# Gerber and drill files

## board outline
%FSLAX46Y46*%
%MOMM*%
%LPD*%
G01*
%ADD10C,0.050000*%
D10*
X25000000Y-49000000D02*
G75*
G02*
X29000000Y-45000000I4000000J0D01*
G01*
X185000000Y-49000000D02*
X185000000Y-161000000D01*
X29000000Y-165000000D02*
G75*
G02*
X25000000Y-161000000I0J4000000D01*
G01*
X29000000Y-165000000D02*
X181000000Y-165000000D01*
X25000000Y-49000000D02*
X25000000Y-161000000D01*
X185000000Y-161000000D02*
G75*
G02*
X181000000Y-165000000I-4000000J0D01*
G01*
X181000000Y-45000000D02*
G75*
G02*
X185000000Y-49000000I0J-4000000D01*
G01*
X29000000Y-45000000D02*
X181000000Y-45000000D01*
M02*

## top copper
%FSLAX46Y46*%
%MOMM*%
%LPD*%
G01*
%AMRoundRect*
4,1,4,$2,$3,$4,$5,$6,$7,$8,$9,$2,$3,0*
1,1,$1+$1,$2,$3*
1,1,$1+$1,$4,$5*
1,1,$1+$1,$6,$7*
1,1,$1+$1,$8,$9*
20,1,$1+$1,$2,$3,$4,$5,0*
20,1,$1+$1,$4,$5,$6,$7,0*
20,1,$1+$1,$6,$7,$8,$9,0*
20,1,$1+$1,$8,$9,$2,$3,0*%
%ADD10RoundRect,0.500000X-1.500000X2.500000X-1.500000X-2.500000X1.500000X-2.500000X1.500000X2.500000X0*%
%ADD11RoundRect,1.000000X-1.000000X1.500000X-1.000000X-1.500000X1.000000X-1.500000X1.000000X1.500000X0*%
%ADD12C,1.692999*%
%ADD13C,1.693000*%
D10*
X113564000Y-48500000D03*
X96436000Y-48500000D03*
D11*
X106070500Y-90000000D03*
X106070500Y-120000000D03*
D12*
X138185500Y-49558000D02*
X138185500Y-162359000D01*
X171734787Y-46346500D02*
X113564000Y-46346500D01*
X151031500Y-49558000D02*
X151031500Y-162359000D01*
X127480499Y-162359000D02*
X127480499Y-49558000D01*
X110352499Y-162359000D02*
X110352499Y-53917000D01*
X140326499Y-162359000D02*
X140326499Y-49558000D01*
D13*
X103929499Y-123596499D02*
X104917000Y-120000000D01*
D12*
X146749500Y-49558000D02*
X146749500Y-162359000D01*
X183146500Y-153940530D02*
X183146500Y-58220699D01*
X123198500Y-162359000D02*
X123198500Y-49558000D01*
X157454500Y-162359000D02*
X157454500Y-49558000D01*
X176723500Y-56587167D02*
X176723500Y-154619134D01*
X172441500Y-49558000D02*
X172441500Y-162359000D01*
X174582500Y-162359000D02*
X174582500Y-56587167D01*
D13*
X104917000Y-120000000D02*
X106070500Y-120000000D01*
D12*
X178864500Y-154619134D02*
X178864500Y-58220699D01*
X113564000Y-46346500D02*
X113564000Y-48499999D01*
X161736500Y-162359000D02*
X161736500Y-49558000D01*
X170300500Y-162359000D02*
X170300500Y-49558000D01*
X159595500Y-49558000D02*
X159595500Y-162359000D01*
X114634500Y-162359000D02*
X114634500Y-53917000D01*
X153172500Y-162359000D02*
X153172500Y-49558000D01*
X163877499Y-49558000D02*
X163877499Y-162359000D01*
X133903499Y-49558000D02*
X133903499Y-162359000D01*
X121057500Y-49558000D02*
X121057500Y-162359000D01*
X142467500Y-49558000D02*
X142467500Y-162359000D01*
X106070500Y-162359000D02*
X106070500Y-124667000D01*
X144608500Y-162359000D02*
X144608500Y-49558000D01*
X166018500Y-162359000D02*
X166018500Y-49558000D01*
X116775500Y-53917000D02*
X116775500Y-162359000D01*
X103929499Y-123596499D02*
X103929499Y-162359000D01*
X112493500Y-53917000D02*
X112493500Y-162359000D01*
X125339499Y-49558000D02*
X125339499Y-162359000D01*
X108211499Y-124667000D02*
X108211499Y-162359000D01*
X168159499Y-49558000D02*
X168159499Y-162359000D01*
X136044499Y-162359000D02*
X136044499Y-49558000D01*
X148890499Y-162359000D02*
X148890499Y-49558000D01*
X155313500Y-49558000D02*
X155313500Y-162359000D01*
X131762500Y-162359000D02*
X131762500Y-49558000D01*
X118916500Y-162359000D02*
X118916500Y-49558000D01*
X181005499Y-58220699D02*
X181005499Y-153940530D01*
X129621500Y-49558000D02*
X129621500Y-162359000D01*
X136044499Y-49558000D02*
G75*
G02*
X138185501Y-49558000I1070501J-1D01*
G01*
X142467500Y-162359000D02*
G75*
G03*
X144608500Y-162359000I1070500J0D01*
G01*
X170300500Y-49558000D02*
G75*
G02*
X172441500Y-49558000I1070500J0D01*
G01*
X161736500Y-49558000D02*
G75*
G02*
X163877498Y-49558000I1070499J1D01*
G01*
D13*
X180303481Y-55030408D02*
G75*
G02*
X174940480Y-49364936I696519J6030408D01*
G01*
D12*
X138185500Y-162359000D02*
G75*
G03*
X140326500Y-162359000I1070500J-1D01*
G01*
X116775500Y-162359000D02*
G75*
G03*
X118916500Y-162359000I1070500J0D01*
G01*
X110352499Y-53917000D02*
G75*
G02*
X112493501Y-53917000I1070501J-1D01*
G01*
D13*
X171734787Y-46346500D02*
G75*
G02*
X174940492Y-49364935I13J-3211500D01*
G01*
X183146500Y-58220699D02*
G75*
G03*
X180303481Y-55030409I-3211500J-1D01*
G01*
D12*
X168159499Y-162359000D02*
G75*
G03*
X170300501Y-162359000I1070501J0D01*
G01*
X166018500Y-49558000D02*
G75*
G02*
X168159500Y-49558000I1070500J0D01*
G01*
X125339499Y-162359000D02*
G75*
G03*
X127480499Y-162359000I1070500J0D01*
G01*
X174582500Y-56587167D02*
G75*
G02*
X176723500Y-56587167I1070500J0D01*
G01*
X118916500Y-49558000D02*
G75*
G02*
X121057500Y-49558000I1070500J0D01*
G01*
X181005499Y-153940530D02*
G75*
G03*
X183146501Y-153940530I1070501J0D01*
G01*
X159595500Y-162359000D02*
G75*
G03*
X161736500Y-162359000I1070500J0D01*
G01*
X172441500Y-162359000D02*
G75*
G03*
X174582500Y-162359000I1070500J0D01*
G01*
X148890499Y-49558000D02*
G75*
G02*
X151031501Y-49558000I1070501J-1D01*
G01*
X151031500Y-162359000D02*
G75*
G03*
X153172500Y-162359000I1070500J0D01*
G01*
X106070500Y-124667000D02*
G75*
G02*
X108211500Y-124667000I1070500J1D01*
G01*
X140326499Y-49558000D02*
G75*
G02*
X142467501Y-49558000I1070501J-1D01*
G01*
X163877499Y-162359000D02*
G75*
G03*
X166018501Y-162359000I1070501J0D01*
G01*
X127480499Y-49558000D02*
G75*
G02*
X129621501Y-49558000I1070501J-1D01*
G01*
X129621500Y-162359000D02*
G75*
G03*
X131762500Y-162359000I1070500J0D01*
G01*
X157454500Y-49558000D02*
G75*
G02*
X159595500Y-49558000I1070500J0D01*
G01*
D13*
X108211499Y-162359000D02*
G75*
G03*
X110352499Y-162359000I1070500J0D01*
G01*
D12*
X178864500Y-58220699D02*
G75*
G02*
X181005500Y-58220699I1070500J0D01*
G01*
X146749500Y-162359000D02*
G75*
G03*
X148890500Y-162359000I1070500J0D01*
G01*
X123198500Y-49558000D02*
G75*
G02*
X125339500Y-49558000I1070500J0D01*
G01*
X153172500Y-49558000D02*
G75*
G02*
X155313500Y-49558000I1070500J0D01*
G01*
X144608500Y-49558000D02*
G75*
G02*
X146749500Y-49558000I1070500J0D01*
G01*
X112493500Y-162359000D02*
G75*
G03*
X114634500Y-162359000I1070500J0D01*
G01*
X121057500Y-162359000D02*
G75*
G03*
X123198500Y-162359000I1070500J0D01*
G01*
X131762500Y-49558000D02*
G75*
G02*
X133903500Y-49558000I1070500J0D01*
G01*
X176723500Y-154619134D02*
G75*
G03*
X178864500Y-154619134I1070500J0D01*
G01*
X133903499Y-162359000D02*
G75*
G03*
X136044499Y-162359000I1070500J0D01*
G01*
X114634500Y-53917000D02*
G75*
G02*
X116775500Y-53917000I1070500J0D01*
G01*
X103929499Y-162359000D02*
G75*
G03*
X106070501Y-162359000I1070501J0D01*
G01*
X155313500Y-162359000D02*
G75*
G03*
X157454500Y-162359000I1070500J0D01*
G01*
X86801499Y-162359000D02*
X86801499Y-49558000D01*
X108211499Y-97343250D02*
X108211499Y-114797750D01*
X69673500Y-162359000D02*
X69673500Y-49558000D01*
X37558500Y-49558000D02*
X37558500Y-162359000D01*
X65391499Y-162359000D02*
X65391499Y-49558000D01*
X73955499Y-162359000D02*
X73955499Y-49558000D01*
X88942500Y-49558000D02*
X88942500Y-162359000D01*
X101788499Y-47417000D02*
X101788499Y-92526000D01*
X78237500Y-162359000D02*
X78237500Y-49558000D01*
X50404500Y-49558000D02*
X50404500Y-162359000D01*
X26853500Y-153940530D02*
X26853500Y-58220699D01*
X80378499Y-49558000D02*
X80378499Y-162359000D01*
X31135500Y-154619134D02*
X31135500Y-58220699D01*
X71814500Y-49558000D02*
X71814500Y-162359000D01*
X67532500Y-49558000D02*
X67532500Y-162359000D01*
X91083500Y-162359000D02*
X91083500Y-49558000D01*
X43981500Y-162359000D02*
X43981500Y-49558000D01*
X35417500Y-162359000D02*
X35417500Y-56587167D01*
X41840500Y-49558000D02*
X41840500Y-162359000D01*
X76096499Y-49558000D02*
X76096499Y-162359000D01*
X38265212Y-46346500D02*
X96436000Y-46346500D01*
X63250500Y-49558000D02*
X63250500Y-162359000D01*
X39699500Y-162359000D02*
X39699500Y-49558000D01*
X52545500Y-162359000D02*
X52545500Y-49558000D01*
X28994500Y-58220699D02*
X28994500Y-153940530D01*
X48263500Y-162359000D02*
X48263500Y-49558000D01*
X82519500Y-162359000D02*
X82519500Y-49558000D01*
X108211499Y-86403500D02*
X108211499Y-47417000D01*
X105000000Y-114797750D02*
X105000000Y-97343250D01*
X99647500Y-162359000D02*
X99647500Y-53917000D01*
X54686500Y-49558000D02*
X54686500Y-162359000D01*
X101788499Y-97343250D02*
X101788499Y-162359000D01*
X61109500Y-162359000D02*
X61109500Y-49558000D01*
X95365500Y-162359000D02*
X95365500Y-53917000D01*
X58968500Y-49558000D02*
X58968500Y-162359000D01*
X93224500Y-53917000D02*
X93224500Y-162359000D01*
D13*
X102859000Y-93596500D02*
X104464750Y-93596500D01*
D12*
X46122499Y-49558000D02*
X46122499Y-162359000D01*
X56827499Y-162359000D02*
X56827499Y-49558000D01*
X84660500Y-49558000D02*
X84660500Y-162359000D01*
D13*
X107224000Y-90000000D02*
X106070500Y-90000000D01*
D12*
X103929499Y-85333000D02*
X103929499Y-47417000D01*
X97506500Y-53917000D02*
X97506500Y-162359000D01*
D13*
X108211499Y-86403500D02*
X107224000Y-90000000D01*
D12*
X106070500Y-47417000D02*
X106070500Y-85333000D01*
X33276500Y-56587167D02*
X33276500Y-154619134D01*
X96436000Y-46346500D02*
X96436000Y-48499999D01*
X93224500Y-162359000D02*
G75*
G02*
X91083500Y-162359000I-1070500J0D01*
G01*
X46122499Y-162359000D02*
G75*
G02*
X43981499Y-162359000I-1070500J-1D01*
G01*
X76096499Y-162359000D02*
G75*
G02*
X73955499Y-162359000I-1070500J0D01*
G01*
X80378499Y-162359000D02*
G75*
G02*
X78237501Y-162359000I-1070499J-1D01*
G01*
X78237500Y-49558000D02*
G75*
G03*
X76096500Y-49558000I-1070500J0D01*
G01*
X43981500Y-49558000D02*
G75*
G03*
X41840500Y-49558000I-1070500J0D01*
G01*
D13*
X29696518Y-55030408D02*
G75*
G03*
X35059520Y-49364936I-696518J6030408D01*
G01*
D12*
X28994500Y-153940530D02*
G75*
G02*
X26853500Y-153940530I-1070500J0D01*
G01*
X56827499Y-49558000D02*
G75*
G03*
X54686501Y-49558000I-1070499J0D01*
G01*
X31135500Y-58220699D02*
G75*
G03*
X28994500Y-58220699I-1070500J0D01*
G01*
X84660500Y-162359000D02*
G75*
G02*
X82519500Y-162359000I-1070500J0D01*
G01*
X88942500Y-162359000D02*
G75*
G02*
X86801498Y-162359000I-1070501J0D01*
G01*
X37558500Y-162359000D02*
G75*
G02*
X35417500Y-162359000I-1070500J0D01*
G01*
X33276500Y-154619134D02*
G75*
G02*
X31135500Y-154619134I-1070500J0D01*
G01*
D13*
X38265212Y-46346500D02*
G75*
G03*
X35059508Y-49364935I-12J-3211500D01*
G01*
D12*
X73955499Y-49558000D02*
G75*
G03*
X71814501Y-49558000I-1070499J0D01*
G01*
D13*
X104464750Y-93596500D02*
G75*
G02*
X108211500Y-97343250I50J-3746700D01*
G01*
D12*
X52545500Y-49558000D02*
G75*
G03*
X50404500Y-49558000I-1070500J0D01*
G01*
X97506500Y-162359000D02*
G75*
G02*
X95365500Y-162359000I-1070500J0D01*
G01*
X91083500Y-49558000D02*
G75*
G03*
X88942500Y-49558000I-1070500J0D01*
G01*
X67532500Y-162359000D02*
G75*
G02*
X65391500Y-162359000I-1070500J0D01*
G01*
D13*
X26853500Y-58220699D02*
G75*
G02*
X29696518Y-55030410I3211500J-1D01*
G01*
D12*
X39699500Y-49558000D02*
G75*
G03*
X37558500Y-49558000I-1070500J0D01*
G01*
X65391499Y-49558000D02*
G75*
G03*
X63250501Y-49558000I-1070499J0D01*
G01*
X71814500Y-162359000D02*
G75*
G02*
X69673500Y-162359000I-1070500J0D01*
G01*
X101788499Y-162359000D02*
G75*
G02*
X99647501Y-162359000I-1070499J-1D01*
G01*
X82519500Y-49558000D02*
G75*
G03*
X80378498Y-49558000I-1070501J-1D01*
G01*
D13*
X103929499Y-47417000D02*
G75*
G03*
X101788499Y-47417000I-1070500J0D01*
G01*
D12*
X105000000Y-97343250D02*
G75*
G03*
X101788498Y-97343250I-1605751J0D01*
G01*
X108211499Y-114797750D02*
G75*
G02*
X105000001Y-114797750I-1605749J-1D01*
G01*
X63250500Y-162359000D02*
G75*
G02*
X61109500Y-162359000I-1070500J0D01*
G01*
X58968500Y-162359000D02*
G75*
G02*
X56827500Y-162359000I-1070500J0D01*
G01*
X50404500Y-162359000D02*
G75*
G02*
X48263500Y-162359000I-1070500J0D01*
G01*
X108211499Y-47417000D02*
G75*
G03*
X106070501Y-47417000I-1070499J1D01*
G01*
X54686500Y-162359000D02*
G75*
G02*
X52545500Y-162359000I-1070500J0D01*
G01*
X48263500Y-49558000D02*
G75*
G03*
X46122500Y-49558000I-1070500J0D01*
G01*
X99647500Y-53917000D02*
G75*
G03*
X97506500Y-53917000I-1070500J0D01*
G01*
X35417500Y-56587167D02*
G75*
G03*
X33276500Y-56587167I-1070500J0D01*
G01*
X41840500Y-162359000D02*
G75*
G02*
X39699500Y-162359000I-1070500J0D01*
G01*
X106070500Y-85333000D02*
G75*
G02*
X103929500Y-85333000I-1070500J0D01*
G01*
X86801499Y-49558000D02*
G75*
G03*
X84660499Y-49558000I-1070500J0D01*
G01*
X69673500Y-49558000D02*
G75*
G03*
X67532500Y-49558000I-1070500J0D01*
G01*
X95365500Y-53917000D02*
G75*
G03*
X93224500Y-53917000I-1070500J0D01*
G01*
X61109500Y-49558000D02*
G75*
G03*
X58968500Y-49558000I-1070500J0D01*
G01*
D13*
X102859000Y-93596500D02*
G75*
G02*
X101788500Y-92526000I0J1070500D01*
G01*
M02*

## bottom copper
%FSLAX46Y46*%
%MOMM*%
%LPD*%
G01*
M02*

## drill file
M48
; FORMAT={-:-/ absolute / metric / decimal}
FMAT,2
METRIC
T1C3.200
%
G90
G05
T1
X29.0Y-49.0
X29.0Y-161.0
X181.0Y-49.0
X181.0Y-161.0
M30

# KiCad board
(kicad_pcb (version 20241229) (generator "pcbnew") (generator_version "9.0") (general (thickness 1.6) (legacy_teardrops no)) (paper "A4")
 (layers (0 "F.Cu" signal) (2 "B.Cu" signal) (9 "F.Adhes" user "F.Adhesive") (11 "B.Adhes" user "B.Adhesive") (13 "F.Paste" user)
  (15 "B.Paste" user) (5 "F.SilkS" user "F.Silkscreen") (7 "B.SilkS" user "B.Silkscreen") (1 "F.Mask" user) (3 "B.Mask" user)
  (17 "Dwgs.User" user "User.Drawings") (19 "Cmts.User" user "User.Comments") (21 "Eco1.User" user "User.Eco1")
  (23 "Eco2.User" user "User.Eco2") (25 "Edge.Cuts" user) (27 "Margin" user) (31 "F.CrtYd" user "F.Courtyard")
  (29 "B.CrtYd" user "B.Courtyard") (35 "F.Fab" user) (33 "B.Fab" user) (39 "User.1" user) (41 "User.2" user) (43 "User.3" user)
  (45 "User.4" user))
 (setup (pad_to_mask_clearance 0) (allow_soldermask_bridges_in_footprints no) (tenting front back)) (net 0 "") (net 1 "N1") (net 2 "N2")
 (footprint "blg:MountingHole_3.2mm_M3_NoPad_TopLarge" (layer "F.Cu") (at 181 49)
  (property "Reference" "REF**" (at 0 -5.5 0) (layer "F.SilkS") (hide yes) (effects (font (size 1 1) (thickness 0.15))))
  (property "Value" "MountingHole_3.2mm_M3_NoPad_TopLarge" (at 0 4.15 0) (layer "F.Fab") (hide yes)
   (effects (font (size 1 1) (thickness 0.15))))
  (pad "" np_thru_hole circle (at 0 0) (size 7.6 7.6) (drill 3.2) (layers) (zone_connect 2)))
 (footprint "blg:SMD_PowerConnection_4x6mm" (layer "F.Cu") (at 113.564 48.5 -90)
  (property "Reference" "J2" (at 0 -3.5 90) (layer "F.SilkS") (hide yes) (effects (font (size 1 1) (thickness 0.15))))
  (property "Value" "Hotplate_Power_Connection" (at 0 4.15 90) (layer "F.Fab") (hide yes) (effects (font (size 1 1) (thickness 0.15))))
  (pad "1" smd roundrect (at 0 0 270) (size 6 4) (layers "F.Cu" "F.Mask" "F.Paste") (roundrect_rratio 0.125) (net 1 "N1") (zone_connect 2)))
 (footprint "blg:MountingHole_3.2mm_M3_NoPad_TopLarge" (layer "F.Cu") (at 29 161)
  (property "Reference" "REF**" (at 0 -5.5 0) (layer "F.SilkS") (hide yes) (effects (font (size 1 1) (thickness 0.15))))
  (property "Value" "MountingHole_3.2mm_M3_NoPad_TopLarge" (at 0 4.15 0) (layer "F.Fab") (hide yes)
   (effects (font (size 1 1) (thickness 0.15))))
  (pad "" np_thru_hole circle (at 0 0) (size 7.6 7.6) (drill 3.2) (layers) (zone_connect 2)))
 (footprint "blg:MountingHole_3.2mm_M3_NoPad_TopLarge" (layer "F.Cu") (at 181 161)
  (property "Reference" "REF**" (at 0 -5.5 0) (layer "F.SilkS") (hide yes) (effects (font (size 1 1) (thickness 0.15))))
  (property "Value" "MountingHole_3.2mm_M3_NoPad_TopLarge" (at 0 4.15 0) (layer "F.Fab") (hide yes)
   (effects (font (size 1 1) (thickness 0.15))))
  (pad "" np_thru_hole circle (at 0 0) (size 7.6 7.6) (drill 3.2) (layers) (zone_connect 2)))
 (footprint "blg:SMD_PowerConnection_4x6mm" (layer "F.Cu") (at 96.436 48.5 -90)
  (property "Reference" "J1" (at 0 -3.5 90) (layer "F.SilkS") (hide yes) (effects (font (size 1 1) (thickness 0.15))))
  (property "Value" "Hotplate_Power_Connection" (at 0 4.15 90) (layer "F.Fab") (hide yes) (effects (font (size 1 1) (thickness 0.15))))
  (pad "1" smd roundrect (at 0 0 270) (size 6 4) (layers "F.Cu" "F.Mask" "F.Paste") (roundrect_rratio 0.125) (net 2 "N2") (zone_connect 2)))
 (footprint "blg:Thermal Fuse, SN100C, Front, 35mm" (layer "F.Cu") (at 106.0705 105 -90)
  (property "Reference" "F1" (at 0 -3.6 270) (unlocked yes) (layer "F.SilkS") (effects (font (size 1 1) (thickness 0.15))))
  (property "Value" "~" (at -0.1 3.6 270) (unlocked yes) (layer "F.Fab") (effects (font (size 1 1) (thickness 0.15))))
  (pad "1" smd roundrect (at -15 0 270) (size 5 4) (layers "F.Cu" "F.Mask") (roundrect_rratio 0.25) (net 2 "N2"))
  (pad "2" smd roundrect (at 15 0 270) (size 5 4) (layers "F.Cu" "F.Mask") (roundrect_rratio 0.25) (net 1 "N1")))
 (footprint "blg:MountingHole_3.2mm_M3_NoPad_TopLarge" (layer "F.Cu") (at 29 49)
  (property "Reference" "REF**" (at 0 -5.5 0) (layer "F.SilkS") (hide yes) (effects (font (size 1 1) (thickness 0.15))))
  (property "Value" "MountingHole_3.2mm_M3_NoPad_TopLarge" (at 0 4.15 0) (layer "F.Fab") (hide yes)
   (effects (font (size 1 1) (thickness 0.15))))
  (pad "" np_thru_hole circle (at 0 0) (size 7.6 7.6) (drill 3.2) (layers) (zone_connect 2)))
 (gr_arc (start 25 49) (mid 26.171573 46.171573) (end 29 45) (stroke (width 0.05) (type solid)) (layer "Edge.Cuts"))
 (gr_line (start 185 49) (end 185 161) (stroke (width 0.05) (type default)) (layer "Edge.Cuts"))
 (gr_arc (start 29 165) (mid 26.171573 163.828427) (end 25 161) (stroke (width 0.05) (type solid)) (layer "Edge.Cuts"))
 (gr_line (start 29 165) (end 181 165) (stroke (width 0.05) (type default)) (layer "Edge.Cuts"))
 (gr_line (start 25 49) (end 25 161) (stroke (width 0.05) (type default)) (layer "Edge.Cuts"))
 (gr_arc (start 185 161) (mid 183.828427 163.828427) (end 181 165) (stroke (width 0.05) (type solid)) (layer "Edge.Cuts"))
 (gr_arc (start 181 45) (mid 183.828427 46.171573) (end 185 49) (stroke (width 0.05) (type solid)) (layer "Edge.Cuts"))
 (gr_line (start 29 45) (end 181 45) (stroke (width 0.05) (type default)) (layer "Edge.Cuts"))
 (segment (start 138.1855 49.558) (end 138.1855 162.359) (width 1.692999) (layer "F.Cu") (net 1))
 (segment (start 171.734787 46.3465) (end 113.564 46.3465) (width 1.692999) (layer "F.Cu") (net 1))
 (segment (start 151.0315 49.558) (end 151.0315 162.359) (width 1.692999) (layer "F.Cu") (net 1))
 (segment (start 127.480499 162.359) (end 127.480499 49.558) (width 1.692999) (layer "F.Cu") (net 1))
 (segment (start 110.352499 162.359) (end 110.352499 53.917) (width 1.692999) (layer "F.Cu") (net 1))
 (segment (start 140.326499 162.359) (end 140.326499 49.558) (width 1.692999) (layer "F.Cu") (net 1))
 (segment (start 103.929499 123.596499) (end 104.917 120) (width 1.693) (layer "F.Cu") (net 1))
 (segment (start 146.7495 49.558) (end 146.7495 162.359) (width 1.692999) (layer "F.Cu") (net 1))
 (segment (start 183.1465 153.94053) (end 183.1465 58.220699) (width 1.692999) (layer "F.Cu") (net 1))
 (segment (start 123.1985 162.359) (end 123.1985 49.558) (width 1.692999) (layer "F.Cu") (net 1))
 (segment (start 157.4545 162.359) (end 157.4545 49.558) (width 1.692999) (layer "F.Cu") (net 1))
 (segment (start 176.7235 56.587167) (end 176.7235 154.619134) (width 1.692999) (layer "F.Cu") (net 1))
 (segment (start 172.4415 49.558) (end 172.4415 162.359) (width 1.692999) (layer "F.Cu") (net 1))
 (segment (start 174.5825 162.359) (end 174.5825 56.587167) (width 1.692999) (layer "F.Cu") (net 1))
 (segment (start 104.917 120) (end 106.0705 120) (width 1.693) (layer "F.Cu") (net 1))
 (segment (start 178.8645 154.619134) (end 178.8645 58.220699) (width 1.692999) (layer "F.Cu") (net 1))
 (segment (start 113.564 46.3465) (end 113.564 48.499999) (width 1.692999) (layer "F.Cu") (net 1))
 (segment (start 161.7365 162.359) (end 161.7365 49.558) (width 1.692999) (layer "F.Cu") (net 1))
 (segment (start 170.3005 162.359) (end 170.3005 49.558) (width 1.692999) (layer "F.Cu") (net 1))
 (segment (start 159.5955 49.558) (end 159.5955 162.359) (width 1.692999) (layer "F.Cu") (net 1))
 (segment (start 114.6345 162.359) (end 114.6345 53.917) (width 1.692999) (layer "F.Cu") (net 1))
 (segment (start 153.1725 162.359) (end 153.1725 49.558) (width 1.692999) (layer "F.Cu") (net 1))
 (segment (start 163.877499 49.558) (end 163.877499 162.359) (width 1.692999) (layer "F.Cu") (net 1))
 (segment (start 133.903499 49.558) (end 133.903499 162.359) (width 1.692999) (layer "F.Cu") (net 1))
 (segment (start 121.0575 49.558) (end 121.0575 162.359) (width 1.692999) (layer "F.Cu") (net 1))
 (segment (start 142.4675 49.558) (end 142.4675 162.359) (width 1.692999) (layer "F.Cu") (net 1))
 (segment (start 106.0705 162.359) (end 106.0705 124.667) (width 1.692999) (layer "F.Cu") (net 1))
 (segment (start 144.6085 162.359) (end 144.6085 49.558) (width 1.692999) (layer "F.Cu") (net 1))
 (segment (start 166.0185 162.359) (end 166.0185 49.558) (width 1.692999) (layer "F.Cu") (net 1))
 (segment (start 116.7755 53.917) (end 116.7755 162.359) (width 1.692999) (layer "F.Cu") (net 1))
 (segment (start 103.929499 123.596499) (end 103.929499 162.359) (width 1.692999) (layer "F.Cu") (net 1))
 (segment (start 112.4935 53.917) (end 112.4935 162.359) (width 1.692999) (layer "F.Cu") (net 1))
 (segment (start 125.339499 49.558) (end 125.339499 162.359) (width 1.692999) (layer "F.Cu") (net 1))
 (segment (start 108.211499 124.667) (end 108.211499 162.359) (width 1.692999) (layer "F.Cu") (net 1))
 (segment (start 168.159499 49.558) (end 168.159499 162.359) (width 1.692999) (layer "F.Cu") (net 1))
 (segment (start 136.044499 162.359) (end 136.044499 49.558) (width 1.692999) (layer "F.Cu") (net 1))
 (segment (start 148.890499 162.359) (end 148.890499 49.558) (width 1.692999) (layer "F.Cu") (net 1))
 (segment (start 155.3135 49.558) (end 155.3135 162.359) (width 1.692999) (layer "F.Cu") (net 1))
 (segment (start 131.7625 162.359) (end 131.7625 49.558) (width 1.692999) (layer "F.Cu") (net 1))
 (segment (start 118.9165 162.359) (end 118.9165 49.558) (width 1.692999) (layer "F.Cu") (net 1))
 (segment (start 181.005499 58.220699) (end 181.005499 153.94053) (width 1.692999) (layer "F.Cu") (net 1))
 (segment (start 129.6215 49.558) (end 129.6215 162.359) (width 1.692999) (layer "F.Cu") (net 1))
 (arc (start 136.044499 49.558) (mid 137.114999 48.4875) (end 138.1855 49.558) (width 1.692999) (layer "F.Cu") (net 1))
 (arc (start 142.4675 162.359) (mid 143.538 163.4295) (end 144.6085 162.359) (width 1.692999) (layer "F.Cu") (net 1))
 (arc (start 170.3005 49.558) (mid 171.371 48.4875) (end 172.4415 49.558) (width 1.692999) (layer "F.Cu") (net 1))
 (arc (start 161.7365 49.558) (mid 162.807 48.4875) (end 163.877499 49.558) (width 1.692999) (layer "F.Cu") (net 1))
 (arc (start 180.303481 55.030408) (mid 176.591438 53.173195) (end 174.940479 49.364936) (width 1.693) (layer "F.Cu") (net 1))
 (arc (start 138.1855 162.359) (mid 139.256 163.4295) (end 140.326499 162.359) (width 1.692999) (layer "F.Cu") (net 1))
 (arc (start 116.7755 162.359) (mid 117.845999 163.4295) (end 118.9165 162.359) (width 1.692999) (layer "F.Cu") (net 1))
 (arc (start 110.352499 53.917) (mid 111.422999 52.8465) (end 112.4935 53.917) (width 1.692999) (layer "F.Cu") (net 1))
 (arc (start 171.734787 46.3465) (mid 173.936344 47.219864) (end 174.940479 49.364936) (width 1.693) (layer "F.Cu") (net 1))
 (arc (start 183.1465 58.220699) (mid 182.220987 55.965041) (end 180.303481 55.030408) (width 1.693) (layer "F.Cu") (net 1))
 (arc (start 168.159499 162.359) (mid 169.23 163.4295) (end 170.3005 162.359) (width 1.692999) (layer "F.Cu") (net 1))
 (arc (start 166.0185 49.558) (mid 167.089 48.4875) (end 168.159499 49.558) (width 1.692999) (layer "F.Cu") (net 1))
 (arc (start 125.339499 162.359) (mid 126.41 163.4295) (end 127.480499 162.359) (width 1.692999) (layer "F.Cu") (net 1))
 (arc (start 174.5825 56.587167) (mid 175.653 55.516667) (end 176.7235 56.587167) (width 1.692999) (layer "F.Cu") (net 1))
 (arc (start 118.9165 49.558) (mid 119.987 48.4875) (end 121.0575 49.558) (width 1.692999) (layer "F.Cu") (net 1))
 (arc (start 181.005499 153.94053) (mid 182.076 155.01103) (end 183.1465 153.94053) (width 1.692999) (layer "F.Cu") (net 1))
 (arc (start 159.5955 162.359) (mid 160.666 163.4295) (end 161.7365 162.359) (width 1.692999) (layer "F.Cu") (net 1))
 (arc (start 172.4415 162.359) (mid 173.512 163.4295) (end 174.5825 162.359) (width 1.692999) (layer "F.Cu") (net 1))
 (arc (start 148.890499 49.558) (mid 149.960999 48.4875) (end 151.0315 49.558) (width 1.692999) (layer "F.Cu") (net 1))
 (arc (start 151.0315 162.359) (mid 152.101999 163.4295) (end 153.1725 162.359) (width 1.692999) (layer "F.Cu") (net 1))
 (arc (start 106.0705 124.667) (mid 107.141 123.596499) (end 108.211499 124.667) (width 1.692999) (layer "F.Cu") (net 1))
 (arc (start 140.326499 49.558) (mid 141.397 48.4875) (end 142.4675 49.558) (width 1.692999) (layer "F.Cu") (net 1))
 (arc (start 163.877499 162.359) (mid 164.947999 163.4295) (end 166.0185 162.359) (width 1.692999) (layer "F.Cu") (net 1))
 (arc (start 127.480499 49.558) (mid 128.550999 48.4875) (end 129.6215 49.558) (width 1.692999) (layer "F.Cu") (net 1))
 (arc (start 129.6215 162.359) (mid 130.692 163.4295) (end 131.7625 162.359) (width 1.692999) (layer "F.Cu") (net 1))
 (arc (start 157.4545 49.558) (mid 158.525 48.4875) (end 159.5955 49.558) (width 1.692999) (layer "F.Cu") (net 1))
 (arc (start 108.211499 162.359) (mid 109.282 163.4295) (end 110.352499 162.359) (width 1.693) (layer "F.Cu") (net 1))
 (arc (start 178.8645 58.220699) (mid 179.934999 57.150199) (end 181.005499 58.220699) (width 1.692999) (layer "F.Cu") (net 1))
 (arc (start 146.7495 162.359) (mid 147.82 163.4295) (end 148.890499 162.359) (width 1.692999) (layer "F.Cu") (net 1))
 (arc (start 123.1985 49.558) (mid 124.268999 48.4875) (end 125.339499 49.558) (width 1.692999) (layer "F.Cu") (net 1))
 (arc (start 153.1725 49.558) (mid 154.243 48.4875) (end 155.3135 49.558) (width 1.692999) (layer "F.Cu") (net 1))
 (arc (start 144.6085 49.558) (mid 145.679 48.4875) (end 146.7495 49.558) (width 1.692999) (layer "F.Cu") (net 1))
 (arc (start 112.4935 162.359) (mid 113.564 163.4295) (end 114.6345 162.359) (width 1.692999) (layer "F.Cu") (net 1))
 (arc (start 121.0575 162.359) (mid 122.128 163.4295) (end 123.1985 162.359) (width 1.692999) (layer "F.Cu") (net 1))
 (arc (start 131.7625 49.558) (mid 132.833 48.4875) (end 133.903499 49.558) (width 1.692999) (layer "F.Cu") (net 1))
 (arc (start 176.7235 154.619134) (mid 177.793999 155.689634) (end 178.8645 154.619134) (width 1.692999) (layer "F.Cu") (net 1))
 (arc (start 133.903499 162.359) (mid 134.974 163.4295) (end 136.044499 162.359) (width 1.692999) (layer "F.Cu") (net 1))
 (arc (start 114.6345 53.917) (mid 115.704999 52.8465) (end 116.7755 53.917) (width 1.692999) (layer "F.Cu") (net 1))
 (arc (start 103.929499 162.359) (mid 105 163.4295) (end 106.0705 162.359) (width 1.692999) (layer "F.Cu") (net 1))
 (arc (start 155.3135 162.359) (mid 156.384 163.4295) (end 157.4545 162.359) (width 1.692999) (layer "F.Cu") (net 1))
 (segment (start 86.801499 162.359) (end 86.801499 49.558) (width 1.692999) (layer "F.Cu") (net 2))
 (segment (start 108.211499 97.34325) (end 108.211499 114.79775) (width 1.692999) (layer "F.Cu") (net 2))
 (segment (start 69.6735 162.359) (end 69.6735 49.558) (width 1.692999) (layer "F.Cu") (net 2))
 (segment (start 37.5585 49.558) (end 37.5585 162.359) (width 1.692999) (layer "F.Cu") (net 2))
 (segment (start 65.391499 162.359) (end 65.391499 49.558) (width 1.692999) (layer "F.Cu") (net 2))
 (segment (start 73.955499 162.359) (end 73.955499 49.558) (width 1.692999) (layer "F.Cu") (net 2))
 (segment (start 88.9425 49.558) (end 88.9425 162.359) (width 1.692999) (layer "F.Cu") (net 2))
 (segment (start 101.788499 47.417) (end 101.788499 92.526) (width 1.692999) (layer "F.Cu") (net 2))
 (segment (start 78.2375 162.359) (end 78.2375 49.558) (width 1.692999) (layer "F.Cu") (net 2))
 (segment (start 50.4045 49.558) (end 50.4045 162.359) (width 1.692999) (layer "F.Cu") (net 2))
 (segment (start 26.8535 153.94053) (end 26.8535 58.220699) (width 1.692999) (layer "F.Cu") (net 2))
 (segment (start 80.378499 49.558) (end 80.378499 162.359) (width 1.692999) (layer "F.Cu") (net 2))
 (segment (start 31.1355 154.619134) (end 31.1355 58.220699) (width 1.692999) (layer "F.Cu") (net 2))
 (segment (start 71.8145 49.558) (end 71.8145 162.359) (width 1.692999) (layer "F.Cu") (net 2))
 (segment (start 67.5325 49.558) (end 67.5325 162.359) (width 1.692999) (layer "F.Cu") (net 2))
 (segment (start 91.0835 162.359) (end 91.0835 49.558) (width 1.692999) (layer "F.Cu") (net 2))
 (segment (start 43.9815 162.359) (end 43.9815 49.558) (width 1.692999) (layer "F.Cu") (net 2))
 (segment (start 35.4175 162.359) (end 35.4175 56.587167) (width 1.692999) (layer "F.Cu") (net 2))
 (segment (start 41.8405 49.558) (end 41.8405 162.359) (width 1.692999) (layer "F.Cu") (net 2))
 (segment (start 76.096499 49.558) (end 76.096499 162.359) (width 1.692999) (layer "F.Cu") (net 2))
 (segment (start 38.265212 46.3465) (end 96.436 46.3465) (width 1.692999) (layer "F.Cu") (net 2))
 (segment (start 63.2505 49.558) (end 63.2505 162.359) (width 1.692999) (layer "F.Cu") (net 2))
 (segment (start 39.6995 162.359) (end 39.6995 49.558) (width 1.692999) (layer "F.Cu") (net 2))
 (segment (start 52.5455 162.359) (end 52.5455 49.558) (width 1.692999) (layer "F.Cu") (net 2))
 (segment (start 28.9945 58.220699) (end 28.9945 153.94053) (width 1.692999) (layer "F.Cu") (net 2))
 (segment (start 48.2635 162.359) (end 48.2635 49.558) (width 1.692999) (layer "F.Cu") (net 2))
 (segment (start 82.5195 162.359) (end 82.5195 49.558) (width 1.692999) (layer "F.Cu") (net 2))
 (segment (start 108.211499 86.4035) (end 108.211499 47.417) (width 1.692999) (layer "F.Cu") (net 2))
 (segment (start 105 114.79775) (end 105 97.34325) (width 1.692999) (layer "F.Cu") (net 2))
 (segment (start 99.6475 162.359) (end 99.6475 53.917) (width 1.692999) (layer "F.Cu") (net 2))
 (segment (start 54.6865 49.558) (end 54.6865 162.359) (width 1.692999) (layer "F.Cu") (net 2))
 (segment (start 101.788499 97.34325) (end 101.788499 162.359) (width 1.692999) (layer "F.Cu") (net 2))
 (segment (start 61.1095 162.359) (end 61.1095 49.558) (width 1.692999) (layer "F.Cu") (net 2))
 (segment (start 95.3655 162.359) (end 95.3655 53.917) (width 1.692999) (layer "F.Cu") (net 2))
 (segment (start 58.9685 49.558) (end 58.9685 162.359) (width 1.692999) (layer "F.Cu") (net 2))
 (segment (start 93.2245 53.917) (end 93.2245 162.359) (width 1.692999) (layer "F.Cu") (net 2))
 (segment (start 102.859 93.5965) (end 104.46475 93.5965) (width 1.693) (layer "F.Cu") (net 2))
 (segment (start 46.122499 49.558) (end 46.122499 162.359) (width 1.692999) (layer "F.Cu") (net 2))
 (segment (start 56.827499 162.359) (end 56.827499 49.558) (width 1.692999) (layer "F.Cu") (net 2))
 (segment (start 84.6605 49.558) (end 84.6605 162.359) (width 1.692999) (layer "F.Cu") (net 2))
 (segment (start 107.224 90) (end 106.0705 90) (width 1.693) (layer "F.Cu") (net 2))
 (segment (start 103.929499 85.333) (end 103.929499 47.417) (width 1.692999) (layer "F.Cu") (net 2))
 (segment (start 97.5065 53.917) (end 97.5065 162.359) (width 1.692999) (layer "F.Cu") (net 2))
 (segment (start 108.211499 86.4035) (end 107.224 90) (width 1.693) (layer "F.Cu") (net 2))
 (segment (start 106.0705 47.417) (end 106.0705 85.333) (width 1.692999) (layer "F.Cu") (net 2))
 (segment (start 33.2765 56.587167) (end 33.2765 154.619134) (width 1.692999) (layer "F.Cu") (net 2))
 (segment (start 96.436 46.3465) (end 96.436 48.499999) (width 1.692999) (layer "F.Cu") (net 2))
 (arc (start 93.2245 162.359) (mid 92.154 163.4295) (end 91.0835 162.359) (width 1.692999) (layer "F.Cu") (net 2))
 (arc (start 46.122499 162.359) (mid 45.051999 163.4295) (end 43.9815 162.359) (width 1.692999) (layer "F.Cu") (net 2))
 (arc (start 76.096499 162.359) (mid 75.026 163.4295) (end 73.955499 162.359) (width 1.692999) (layer "F.Cu") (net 2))
 (arc (start 80.378499 162.359) (mid 79.308 163.4295) (end 78.2375 162.359) (width 1.692999) (layer "F.Cu") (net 2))
 (arc (start 78.2375 49.558) (mid 77.167 48.4875) (end 76.096499 49.558) (width 1.692999) (layer "F.Cu") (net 2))
 (arc (start 43.9815 49.558) (mid 42.910999 48.4875) (end 41.8405 49.558) (width 1.692999) (layer "F.Cu") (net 2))
 (arc (start 29.696518 55.030408) (mid 33.408561 53.173195) (end 35.05952 49.364936) (width 1.693) (layer "F.Cu") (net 2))
 (arc (start 28.9945 153.94053) (mid 27.923999 155.01103) (end 26.8535 153.94053) (width 1.692999) (layer "F.Cu") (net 2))
 (arc (start 56.827499 49.558) (mid 55.756999 48.4875) (end 54.6865 49.558) (width 1.692999) (layer "F.Cu") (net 2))
 (arc (start 31.1355 58.220699) (mid 30.064999 57.150199) (end 28.9945 58.220699) (width 1.692999) (layer "F.Cu") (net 2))
 (arc (start 84.6605 162.359) (mid 83.59 163.4295) (end 82.5195 162.359) (width 1.692999) (layer "F.Cu") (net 2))
 (arc (start 88.9425 162.359) (mid 87.871999 163.4295) (end 86.801499 162.359) (width 1.692999) (layer "F.Cu") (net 2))
 (arc (start 37.5585 162.359) (mid 36.488 163.4295) (end 35.4175 162.359) (width 1.692999) (layer "F.Cu") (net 2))
 (arc (start 33.2765 154.619134) (mid 32.205999 155.689634) (end 31.1355 154.619134) (width 1.692999) (layer "F.Cu") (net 2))
 (arc (start 38.265212 46.3465) (mid 36.063655 47.219864) (end 35.05952 49.364936) (width 1.693) (layer "F.Cu") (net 2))
 (arc (start 73.955499 49.558) (mid 72.884999 48.4875) (end 71.8145 49.558) (width 1.692999) (layer "F.Cu") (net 2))
 (arc (start 104.46475 93.5965) (mid 107.114102 94.693897) (end 108.211499 97.34325) (width 1.693) (layer "F.Cu") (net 2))
 (arc (start 52.5455 49.558) (mid 51.475 48.4875) (end 50.4045 49.558) (width 1.692999) (layer "F.Cu") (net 2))
 (arc (start 97.5065 162.359) (mid 96.436 163.4295) (end 95.3655 162.359) (width 1.692999) (layer "F.Cu") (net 2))
 (arc (start 91.0835 49.558) (mid 90.012999 48.4875) (end 88.9425 49.558) (width 1.692999) (layer "F.Cu") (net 2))
 (arc (start 67.5325 162.359) (mid 66.461999 163.4295) (end 65.391499 162.359) (width 1.692999) (layer "F.Cu") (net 2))
 (arc (start 26.8535 58.220699) (mid 27.779012 55.965041) (end 29.696518 55.030408) (width 1.693) (layer "F.Cu") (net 2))
 (arc (start 39.6995 49.558) (mid 38.629 48.4875) (end 37.5585 49.558) (width 1.692999) (layer "F.Cu") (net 2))
 (arc (start 65.391499 49.558) (mid 64.321 48.4875) (end 63.2505 49.558) (width 1.692999) (layer "F.Cu") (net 2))
 (arc (start 71.8145 162.359) (mid 70.744 163.4295) (end 69.6735 162.359) (width 1.692999) (layer "F.Cu") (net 2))
 (arc (start 101.788499 162.359) (mid 100.718 163.4295) (end 99.6475 162.359) (width 1.692999) (layer "F.Cu") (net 2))
 (arc (start 82.5195 49.558) (mid 81.449 48.4875) (end 80.378499 49.558) (width 1.692999) (layer "F.Cu") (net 2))
 (arc (start 103.929499 47.417) (mid 102.859 46.3465) (end 101.788499 47.417) (width 1.693) (layer "F.Cu") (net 2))
 (arc (start 105 97.34325) (mid 103.39425 95.737499) (end 101.788499 97.34325) (width 1.692999) (layer "F.Cu") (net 2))
 (arc (start 108.211499 114.79775) (mid 106.60575 116.4035) (end 105 114.79775) (width 1.692999) (layer "F.Cu") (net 2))
 (arc (start 63.2505 162.359) (mid 62.18 163.4295) (end 61.1095 162.359) (width 1.692999) (layer "F.Cu") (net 2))
 (arc (start 58.9685 162.359) (mid 57.897999 163.4295) (end 56.827499 162.359) (width 1.692999) (layer "F.Cu") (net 2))
 (arc (start 50.4045 162.359) (mid 49.333999 163.4295) (end 48.2635 162.359) (width 1.692999) (layer "F.Cu") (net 2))
 (arc (start 108.211499 47.417) (mid 107.141 46.3465) (end 106.0705 47.417) (width 1.692999) (layer "F.Cu") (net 2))
 (arc (start 54.6865 162.359) (mid 53.616 163.4295) (end 52.5455 162.359) (width 1.692999) (layer "F.Cu") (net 2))
 (arc (start 48.2635 49.558) (mid 47.193 48.4875) (end 46.122499 49.558) (width 1.692999) (layer "F.Cu") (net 2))
 (arc (start 99.6475 53.917) (mid 98.577 52.8465) (end 97.5065 53.917) (width 1.692999) (layer "F.Cu") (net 2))
 (arc (start 35.4175 56.587167) (mid 34.346999 55.516667) (end 33.2765 56.587167) (width 1.692999) (layer "F.Cu") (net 2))
 (arc (start 41.8405 162.359) (mid 40.77 163.4295) (end 39.6995 162.359) (width 1.692999) (layer "F.Cu") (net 2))
 (arc (start 106.0705 85.333) (mid 105 86.4035) (end 103.929499 85.333) (width 1.692999) (layer "F.Cu") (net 2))
 (arc (start 86.801499 49.558) (mid 85.731 48.4875) (end 84.6605 49.558) (width 1.692999) (layer "F.Cu") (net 2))
 (arc (start 69.6735 49.558) (mid 68.603 48.4875) (end 67.5325 49.558) (width 1.692999) (layer "F.Cu") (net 2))
 (arc (start 95.3655 53.917) (mid 94.294999 52.8465) (end 93.2245 53.917) (width 1.692999) (layer "F.Cu") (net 2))
 (arc (start 61.1095 49.558) (mid 60.038999 48.4875) (end 58.9685 49.558) (width 1.692999) (layer "F.Cu") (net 2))
 (arc (start 102.859 93.5965) (mid 102.102042 93.282957) (end 101.788499 92.526) (width 1.693) (layer "F.Cu") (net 2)))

